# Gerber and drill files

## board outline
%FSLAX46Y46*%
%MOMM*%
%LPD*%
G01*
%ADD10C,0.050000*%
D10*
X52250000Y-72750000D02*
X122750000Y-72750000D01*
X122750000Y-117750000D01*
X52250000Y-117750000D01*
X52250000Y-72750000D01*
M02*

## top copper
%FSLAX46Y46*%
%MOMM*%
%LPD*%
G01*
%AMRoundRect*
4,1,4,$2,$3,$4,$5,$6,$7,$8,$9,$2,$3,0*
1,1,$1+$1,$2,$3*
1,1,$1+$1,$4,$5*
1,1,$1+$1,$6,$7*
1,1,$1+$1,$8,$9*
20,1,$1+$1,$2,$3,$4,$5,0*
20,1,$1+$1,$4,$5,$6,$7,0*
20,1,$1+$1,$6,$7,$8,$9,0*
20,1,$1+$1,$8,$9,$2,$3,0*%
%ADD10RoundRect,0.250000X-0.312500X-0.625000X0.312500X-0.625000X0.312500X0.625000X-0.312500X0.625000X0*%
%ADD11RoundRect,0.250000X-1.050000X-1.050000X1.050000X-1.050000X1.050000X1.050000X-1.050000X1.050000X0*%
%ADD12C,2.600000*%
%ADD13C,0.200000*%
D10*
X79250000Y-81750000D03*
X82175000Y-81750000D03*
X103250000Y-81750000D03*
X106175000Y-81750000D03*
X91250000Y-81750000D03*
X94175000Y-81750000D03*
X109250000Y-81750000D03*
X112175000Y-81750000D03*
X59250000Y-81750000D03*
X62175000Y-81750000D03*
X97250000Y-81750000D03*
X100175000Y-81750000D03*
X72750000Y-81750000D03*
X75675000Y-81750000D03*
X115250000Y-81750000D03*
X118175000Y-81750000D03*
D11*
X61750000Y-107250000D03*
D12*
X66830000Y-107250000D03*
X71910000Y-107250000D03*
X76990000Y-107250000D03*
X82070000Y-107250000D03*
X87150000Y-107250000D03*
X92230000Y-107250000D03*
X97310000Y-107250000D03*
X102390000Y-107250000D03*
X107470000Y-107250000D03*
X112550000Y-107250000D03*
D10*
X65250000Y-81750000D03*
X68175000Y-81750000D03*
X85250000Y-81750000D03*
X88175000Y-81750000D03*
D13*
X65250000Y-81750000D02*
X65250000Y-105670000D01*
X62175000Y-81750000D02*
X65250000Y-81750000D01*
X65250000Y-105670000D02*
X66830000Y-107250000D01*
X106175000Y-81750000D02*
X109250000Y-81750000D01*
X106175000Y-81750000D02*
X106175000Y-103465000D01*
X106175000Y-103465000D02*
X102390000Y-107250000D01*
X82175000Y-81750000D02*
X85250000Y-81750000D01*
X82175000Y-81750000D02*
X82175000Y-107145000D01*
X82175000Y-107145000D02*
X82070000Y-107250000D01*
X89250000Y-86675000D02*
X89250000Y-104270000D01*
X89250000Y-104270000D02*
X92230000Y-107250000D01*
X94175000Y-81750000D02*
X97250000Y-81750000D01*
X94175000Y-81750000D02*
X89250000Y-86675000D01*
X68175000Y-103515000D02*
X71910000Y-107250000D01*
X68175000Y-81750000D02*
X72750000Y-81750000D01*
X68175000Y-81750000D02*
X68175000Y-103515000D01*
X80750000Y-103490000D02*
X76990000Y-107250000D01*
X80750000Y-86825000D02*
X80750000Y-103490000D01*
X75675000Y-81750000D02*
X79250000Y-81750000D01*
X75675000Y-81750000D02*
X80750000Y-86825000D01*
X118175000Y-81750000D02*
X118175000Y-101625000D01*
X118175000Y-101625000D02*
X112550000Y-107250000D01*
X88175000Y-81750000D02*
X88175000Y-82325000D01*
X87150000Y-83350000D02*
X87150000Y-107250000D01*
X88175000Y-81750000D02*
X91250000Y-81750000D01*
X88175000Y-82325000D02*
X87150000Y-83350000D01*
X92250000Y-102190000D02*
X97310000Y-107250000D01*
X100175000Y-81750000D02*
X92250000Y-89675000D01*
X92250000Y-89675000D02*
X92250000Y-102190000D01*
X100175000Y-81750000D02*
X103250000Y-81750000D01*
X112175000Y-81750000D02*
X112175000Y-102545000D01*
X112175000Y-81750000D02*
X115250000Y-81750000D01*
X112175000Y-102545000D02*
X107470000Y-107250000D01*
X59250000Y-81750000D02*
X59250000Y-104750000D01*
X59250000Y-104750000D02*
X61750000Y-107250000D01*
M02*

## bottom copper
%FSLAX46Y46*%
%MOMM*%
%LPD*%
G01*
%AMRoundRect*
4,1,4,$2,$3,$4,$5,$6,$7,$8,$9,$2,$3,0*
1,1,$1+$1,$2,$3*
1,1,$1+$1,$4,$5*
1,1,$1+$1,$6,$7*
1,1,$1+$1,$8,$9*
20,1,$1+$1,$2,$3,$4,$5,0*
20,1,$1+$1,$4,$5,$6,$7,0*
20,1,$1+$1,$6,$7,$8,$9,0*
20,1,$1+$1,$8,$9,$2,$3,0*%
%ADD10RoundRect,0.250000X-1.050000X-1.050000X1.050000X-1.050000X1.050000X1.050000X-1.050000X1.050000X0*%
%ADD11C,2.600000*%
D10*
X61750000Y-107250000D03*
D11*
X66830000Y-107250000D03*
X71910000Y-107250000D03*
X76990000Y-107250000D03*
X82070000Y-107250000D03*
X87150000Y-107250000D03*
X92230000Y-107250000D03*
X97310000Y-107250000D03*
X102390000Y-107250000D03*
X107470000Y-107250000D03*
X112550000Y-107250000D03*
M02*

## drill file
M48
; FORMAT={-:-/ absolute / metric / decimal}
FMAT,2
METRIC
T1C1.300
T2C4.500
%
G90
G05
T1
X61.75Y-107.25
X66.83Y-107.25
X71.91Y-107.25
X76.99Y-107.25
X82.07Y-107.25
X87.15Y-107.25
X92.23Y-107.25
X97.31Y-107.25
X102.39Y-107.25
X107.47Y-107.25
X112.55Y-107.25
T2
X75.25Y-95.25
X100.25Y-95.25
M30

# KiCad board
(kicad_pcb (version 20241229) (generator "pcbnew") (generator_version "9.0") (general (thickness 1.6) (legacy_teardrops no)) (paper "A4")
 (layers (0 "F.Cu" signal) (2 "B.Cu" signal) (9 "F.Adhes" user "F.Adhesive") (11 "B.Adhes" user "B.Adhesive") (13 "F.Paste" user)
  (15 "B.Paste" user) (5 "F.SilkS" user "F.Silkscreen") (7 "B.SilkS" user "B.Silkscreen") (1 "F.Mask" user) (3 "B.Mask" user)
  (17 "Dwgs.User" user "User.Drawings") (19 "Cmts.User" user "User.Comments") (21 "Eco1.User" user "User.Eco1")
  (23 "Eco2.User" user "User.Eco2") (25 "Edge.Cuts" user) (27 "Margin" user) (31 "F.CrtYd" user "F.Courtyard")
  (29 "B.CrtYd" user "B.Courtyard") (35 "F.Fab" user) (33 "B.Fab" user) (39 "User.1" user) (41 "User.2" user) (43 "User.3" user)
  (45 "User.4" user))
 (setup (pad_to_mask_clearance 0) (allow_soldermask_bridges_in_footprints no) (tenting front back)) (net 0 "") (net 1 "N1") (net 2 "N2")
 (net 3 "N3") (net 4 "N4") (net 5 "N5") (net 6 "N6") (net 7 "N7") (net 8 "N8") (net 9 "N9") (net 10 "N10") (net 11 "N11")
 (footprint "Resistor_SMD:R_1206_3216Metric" (layer "F.Cu") (at 80.7125 81.75)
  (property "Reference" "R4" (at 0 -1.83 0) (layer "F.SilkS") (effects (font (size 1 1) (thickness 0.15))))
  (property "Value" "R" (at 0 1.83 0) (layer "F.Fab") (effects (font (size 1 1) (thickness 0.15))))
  (pad "1" smd roundrect (at -1.4625 0) (size 1.125 1.75) (layers "F.Cu" "F.Mask" "F.Paste") (roundrect_rratio 0.222222) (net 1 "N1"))
  (pad "2" smd roundrect (at 1.4625 0) (size 1.125 1.75) (layers "F.Cu" "F.Mask" "F.Paste") (roundrect_rratio 0.222222) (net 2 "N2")))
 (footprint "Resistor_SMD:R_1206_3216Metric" (layer "F.Cu") (at 104.7125 81.75)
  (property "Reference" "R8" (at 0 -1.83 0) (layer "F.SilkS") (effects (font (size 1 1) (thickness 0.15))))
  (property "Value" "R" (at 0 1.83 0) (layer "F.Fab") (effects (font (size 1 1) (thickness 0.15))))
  (pad "1" smd roundrect (at -1.4625 0) (size 1.125 1.75) (layers "F.Cu" "F.Mask" "F.Paste") (roundrect_rratio 0.222222) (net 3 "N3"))
  (pad "2" smd roundrect (at 1.4625 0) (size 1.125 1.75) (layers "F.Cu" "F.Mask" "F.Paste") (roundrect_rratio 0.222222) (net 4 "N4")))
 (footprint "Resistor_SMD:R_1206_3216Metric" (layer "F.Cu") (at 92.7125 81.75)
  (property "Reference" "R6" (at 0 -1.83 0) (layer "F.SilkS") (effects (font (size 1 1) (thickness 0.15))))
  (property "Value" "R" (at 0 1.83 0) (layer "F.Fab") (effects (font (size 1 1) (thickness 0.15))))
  (pad "1" smd roundrect (at -1.4625 0) (size 1.125 1.75) (layers "F.Cu" "F.Mask" "F.Paste") (roundrect_rratio 0.222222) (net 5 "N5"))
  (pad "2" smd roundrect (at 1.4625 0) (size 1.125 1.75) (layers "F.Cu" "F.Mask" "F.Paste") (roundrect_rratio 0.222222) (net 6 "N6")))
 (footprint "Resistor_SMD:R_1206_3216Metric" (layer "F.Cu") (at 110.7125 81.75)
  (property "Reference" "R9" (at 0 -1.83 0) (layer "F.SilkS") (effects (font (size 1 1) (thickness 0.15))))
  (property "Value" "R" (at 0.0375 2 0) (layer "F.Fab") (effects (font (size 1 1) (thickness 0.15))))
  (pad "1" smd roundrect (at -1.4625 0) (size 1.125 1.75) (layers "F.Cu" "F.Mask" "F.Paste") (roundrect_rratio 0.222222) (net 4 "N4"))
  (pad "2" smd roundrect (at 1.4625 0) (size 1.125 1.75) (layers "F.Cu" "F.Mask" "F.Paste") (roundrect_rratio 0.222222) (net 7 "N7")))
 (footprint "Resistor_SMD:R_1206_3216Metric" (layer "F.Cu") (at 60.7125 81.75)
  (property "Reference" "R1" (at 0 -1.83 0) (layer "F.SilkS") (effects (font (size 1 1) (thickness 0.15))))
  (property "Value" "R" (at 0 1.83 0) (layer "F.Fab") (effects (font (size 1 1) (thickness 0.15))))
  (pad "1" smd roundrect (at -1.4625 0) (size 1.125 1.75) (layers "F.Cu" "F.Mask" "F.Paste") (roundrect_rratio 0.222222) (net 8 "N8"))
  (pad "2" smd roundrect (at 1.4625 0) (size 1.125 1.75) (layers "F.Cu" "F.Mask" "F.Paste") (roundrect_rratio 0.222222) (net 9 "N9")))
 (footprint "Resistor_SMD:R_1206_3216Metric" (layer "F.Cu") (at 98.7125 81.75)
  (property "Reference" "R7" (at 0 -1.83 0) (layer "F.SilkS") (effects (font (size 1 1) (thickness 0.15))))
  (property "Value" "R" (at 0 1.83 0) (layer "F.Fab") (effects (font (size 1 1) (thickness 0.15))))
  (pad "1" smd roundrect (at -1.4625 0) (size 1.125 1.75) (layers "F.Cu" "F.Mask" "F.Paste") (roundrect_rratio 0.222222) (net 6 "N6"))
  (pad "2" smd roundrect (at 1.4625 0) (size 1.125 1.75) (layers "F.Cu" "F.Mask" "F.Paste") (roundrect_rratio 0.222222) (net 3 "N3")))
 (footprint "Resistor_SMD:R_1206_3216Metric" (layer "F.Cu") (at 74.2125 81.75)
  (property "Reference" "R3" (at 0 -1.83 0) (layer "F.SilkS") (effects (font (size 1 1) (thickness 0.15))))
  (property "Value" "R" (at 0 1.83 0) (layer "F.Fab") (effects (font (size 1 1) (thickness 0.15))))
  (pad "1" smd roundrect (at -1.4625 0) (size 1.125 1.75) (layers "F.Cu" "F.Mask" "F.Paste") (roundrect_rratio 0.222222) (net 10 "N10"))
  (pad "2" smd roundrect (at 1.4625 0) (size 1.125 1.75) (layers "F.Cu" "F.Mask" "F.Paste") (roundrect_rratio 0.222222) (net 1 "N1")))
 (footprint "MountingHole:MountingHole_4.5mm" (layer "F.Cu") (at 75.25 95.25 90)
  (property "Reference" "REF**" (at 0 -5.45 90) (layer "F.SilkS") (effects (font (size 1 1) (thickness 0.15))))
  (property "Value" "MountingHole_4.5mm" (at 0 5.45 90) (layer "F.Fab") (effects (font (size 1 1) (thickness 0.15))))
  (pad "" np_thru_hole circle (at 0 0 90) (size 4.5 4.5) (drill 4.5) (layers "*.Cu" "*.Mask")))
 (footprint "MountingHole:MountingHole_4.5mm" (layer "F.Cu") (at 100.25 95.25 90)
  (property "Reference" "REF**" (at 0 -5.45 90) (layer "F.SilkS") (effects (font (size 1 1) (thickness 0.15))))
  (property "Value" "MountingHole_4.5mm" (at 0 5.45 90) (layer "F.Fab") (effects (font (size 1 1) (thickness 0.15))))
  (pad "" np_thru_hole circle (at 0 0 90) (size 4.5 4.5) (drill 4.5) (layers "*.Cu" "*.Mask")))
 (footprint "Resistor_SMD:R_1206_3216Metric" (layer "F.Cu") (at 116.7125 81.75)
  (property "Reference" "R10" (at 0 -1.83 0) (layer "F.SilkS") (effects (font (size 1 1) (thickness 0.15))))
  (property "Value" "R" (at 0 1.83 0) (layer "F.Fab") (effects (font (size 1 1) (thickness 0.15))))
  (pad "1" smd roundrect (at -1.4625 0) (size 1.125 1.75) (layers "F.Cu" "F.Mask" "F.Paste") (roundrect_rratio 0.222222) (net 7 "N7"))
  (pad "2" smd roundrect (at 1.4625 0) (size 1.125 1.75) (layers "F.Cu" "F.Mask" "F.Paste") (roundrect_rratio 0.222222) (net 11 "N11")))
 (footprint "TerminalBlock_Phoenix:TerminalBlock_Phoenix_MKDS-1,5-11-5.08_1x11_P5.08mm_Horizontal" (layer "F.Cu") (at 61.75 107.25)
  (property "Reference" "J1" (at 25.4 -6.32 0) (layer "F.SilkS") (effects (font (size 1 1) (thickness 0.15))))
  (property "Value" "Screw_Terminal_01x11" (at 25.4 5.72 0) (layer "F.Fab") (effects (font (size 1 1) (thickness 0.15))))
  (pad "1" thru_hole roundrect (at 0 0) (size 2.6 2.6) (drill 1.3) (layers "*.Cu" "*.Mask") (remove_unused_layers no)
   (roundrect_rratio 0.096154) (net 8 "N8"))
  (pad "2" thru_hole circle (at 5.08 0) (size 2.6 2.6) (drill 1.3) (layers "*.Cu" "*.Mask") (remove_unused_layers no) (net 9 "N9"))
  (pad "3" thru_hole circle (at 10.16 0) (size 2.6 2.6) (drill 1.3) (layers "*.Cu" "*.Mask") (remove_unused_layers no) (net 10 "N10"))
  (pad "4" thru_hole circle (at 15.24 0) (size 2.6 2.6) (drill 1.3) (layers "*.Cu" "*.Mask") (remove_unused_layers no) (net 1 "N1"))
  (pad "5" thru_hole circle (at 20.32 0) (size 2.6 2.6) (drill 1.3) (layers "*.Cu" "*.Mask") (remove_unused_layers no) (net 2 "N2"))
  (pad "6" thru_hole circle (at 25.4 0) (size 2.6 2.6) (drill 1.3) (layers "*.Cu" "*.Mask") (remove_unused_layers no) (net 5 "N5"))
  (pad "7" thru_hole circle (at 30.48 0) (size 2.6 2.6) (drill 1.3) (layers "*.Cu" "*.Mask") (remove_unused_layers no) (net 6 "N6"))
  (pad "8" thru_hole circle (at 35.56 0) (size 2.6 2.6) (drill 1.3) (layers "*.Cu" "*.Mask") (remove_unused_layers no) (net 3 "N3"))
  (pad "9" thru_hole circle (at 40.64 0) (size 2.6 2.6) (drill 1.3) (layers "*.Cu" "*.Mask") (remove_unused_layers no) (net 4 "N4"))
  (pad "10" thru_hole circle (at 45.72 0) (size 2.6 2.6) (drill 1.3) (layers "*.Cu" "*.Mask") (remove_unused_layers no) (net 7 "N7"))
  (pad "11" thru_hole circle (at 50.8 0) (size 2.6 2.6) (drill 1.3) (layers "*.Cu" "*.Mask") (remove_unused_layers no) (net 11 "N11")))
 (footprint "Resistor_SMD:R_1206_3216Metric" (layer "F.Cu") (at 66.7125 81.75)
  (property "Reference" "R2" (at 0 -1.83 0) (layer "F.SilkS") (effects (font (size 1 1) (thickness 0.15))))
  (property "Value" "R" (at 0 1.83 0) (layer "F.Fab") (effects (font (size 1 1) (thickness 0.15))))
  (pad "1" smd roundrect (at -1.4625 0) (size 1.125 1.75) (layers "F.Cu" "F.Mask" "F.Paste") (roundrect_rratio 0.222222) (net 9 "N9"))
  (pad "2" smd roundrect (at 1.4625 0) (size 1.125 1.75) (layers "F.Cu" "F.Mask" "F.Paste") (roundrect_rratio 0.222222) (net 10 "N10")))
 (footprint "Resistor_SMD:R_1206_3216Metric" (layer "F.Cu") (at 86.7125 81.75)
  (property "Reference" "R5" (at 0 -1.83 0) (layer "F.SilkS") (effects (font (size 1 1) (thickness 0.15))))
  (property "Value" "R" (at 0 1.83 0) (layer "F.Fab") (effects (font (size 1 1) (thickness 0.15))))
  (pad "1" smd roundrect (at -1.4625 0) (size 1.125 1.75) (layers "F.Cu" "F.Mask" "F.Paste") (roundrect_rratio 0.222222) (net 2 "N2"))
  (pad "2" smd roundrect (at 1.4625 0) (size 1.125 1.75) (layers "F.Cu" "F.Mask" "F.Paste") (roundrect_rratio 0.222222) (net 5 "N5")))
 (gr_rect (start 52.25 72.75) (end 122.75 117.75) (stroke (width 0.05) (type default)) (fill no) (layer "Edge.Cuts"))
 (segment (start 65.25 81.75) (end 65.25 105.67) (width 0.2) (layer "F.Cu") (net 9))
 (segment (start 62.175 81.75) (end 65.25 81.75) (width 0.2) (layer "F.Cu") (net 9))
 (segment (start 65.25 105.67) (end 66.83 107.25) (width 0.2) (layer "F.Cu") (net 9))
 (segment (start 106.175 81.75) (end 109.25 81.75) (width 0.2) (layer "F.Cu") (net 4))
 (segment (start 106.175 81.75) (end 106.175 103.465) (width 0.2) (layer "F.Cu") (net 4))
 (segment (start 106.175 103.465) (end 102.39 107.25) (width 0.2) (layer "F.Cu") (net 4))
 (segment (start 82.175 81.75) (end 85.25 81.75) (width 0.2) (layer "F.Cu") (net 2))
 (segment (start 82.175 81.75) (end 82.175 107.145) (width 0.2) (layer "F.Cu") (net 2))
 (segment (start 82.175 107.145) (end 82.07 107.25) (width 0.2) (layer "F.Cu") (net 2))
 (segment (start 89.25 86.675) (end 89.25 104.27) (width 0.2) (layer "F.Cu") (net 6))
 (segment (start 89.25 104.27) (end 92.23 107.25) (width 0.2) (layer "F.Cu") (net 6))
 (segment (start 94.175 81.75) (end 97.25 81.75) (width 0.2) (layer "F.Cu") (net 6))
 (segment (start 94.175 81.75) (end 89.25 86.675) (width 0.2) (layer "F.Cu") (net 6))
 (segment (start 68.175 103.515) (end 71.91 107.25) (width 0.2) (layer "F.Cu") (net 10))
 (segment (start 68.175 81.75) (end 72.75 81.75) (width 0.2) (layer "F.Cu") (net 10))
 (segment (start 68.175 81.75) (end 68.175 103.515) (width 0.2) (layer "F.Cu") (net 10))
 (segment (start 80.75 103.49) (end 76.99 107.25) (width 0.2) (layer "F.Cu") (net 1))
 (segment (start 80.75 86.825) (end 80.75 103.49) (width 0.2) (layer "F.Cu") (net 1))
 (segment (start 75.675 81.75) (end 79.25 81.75) (width 0.2) (layer "F.Cu") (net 1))
 (segment (start 75.675 81.75) (end 80.75 86.825) (width 0.2) (layer "F.Cu") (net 1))
 (segment (start 118.175 81.75) (end 118.175 101.625) (width 0.2) (layer "F.Cu") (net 11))
 (segment (start 118.175 101.625) (end 112.55 107.25) (width 0.2) (layer "F.Cu") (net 11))
 (segment (start 88.175 81.75) (end 88.175 82.325) (width 0.2) (layer "F.Cu") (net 5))
 (segment (start 87.15 83.35) (end 87.15 107.25) (width 0.2) (layer "F.Cu") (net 5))
 (segment (start 88.175 81.75) (end 91.25 81.75) (width 0.2) (layer "F.Cu") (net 5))
 (segment (start 88.175 82.325) (end 87.15 83.35) (width 0.2) (layer "F.Cu") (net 5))
 (segment (start 92.25 102.19) (end 97.31 107.25) (width 0.2) (layer "F.Cu") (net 3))
 (segment (start 100.175 81.75) (end 92.25 89.675) (width 0.2) (layer "F.Cu") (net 3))
 (segment (start 92.25 89.675) (end 92.25 102.19) (width 0.2) (layer "F.Cu") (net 3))
 (segment (start 100.175 81.75) (end 103.25 81.75) (width 0.2) (layer "F.Cu") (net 3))
 (segment (start 112.175 81.75) (end 112.175 102.545) (width 0.2) (layer "F.Cu") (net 7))
 (segment (start 112.175 81.75) (end 115.25 81.75) (width 0.2) (layer "F.Cu") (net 7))
 (segment (start 112.175 102.545) (end 107.47 107.25) (width 0.2) (layer "F.Cu") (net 7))
 (segment (start 59.25 81.75) (end 59.25 104.75) (width 0.2) (layer "F.Cu") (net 8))
 (segment (start 59.25 104.75) (end 61.75 107.25) (width 0.2) (layer "F.Cu") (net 8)))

